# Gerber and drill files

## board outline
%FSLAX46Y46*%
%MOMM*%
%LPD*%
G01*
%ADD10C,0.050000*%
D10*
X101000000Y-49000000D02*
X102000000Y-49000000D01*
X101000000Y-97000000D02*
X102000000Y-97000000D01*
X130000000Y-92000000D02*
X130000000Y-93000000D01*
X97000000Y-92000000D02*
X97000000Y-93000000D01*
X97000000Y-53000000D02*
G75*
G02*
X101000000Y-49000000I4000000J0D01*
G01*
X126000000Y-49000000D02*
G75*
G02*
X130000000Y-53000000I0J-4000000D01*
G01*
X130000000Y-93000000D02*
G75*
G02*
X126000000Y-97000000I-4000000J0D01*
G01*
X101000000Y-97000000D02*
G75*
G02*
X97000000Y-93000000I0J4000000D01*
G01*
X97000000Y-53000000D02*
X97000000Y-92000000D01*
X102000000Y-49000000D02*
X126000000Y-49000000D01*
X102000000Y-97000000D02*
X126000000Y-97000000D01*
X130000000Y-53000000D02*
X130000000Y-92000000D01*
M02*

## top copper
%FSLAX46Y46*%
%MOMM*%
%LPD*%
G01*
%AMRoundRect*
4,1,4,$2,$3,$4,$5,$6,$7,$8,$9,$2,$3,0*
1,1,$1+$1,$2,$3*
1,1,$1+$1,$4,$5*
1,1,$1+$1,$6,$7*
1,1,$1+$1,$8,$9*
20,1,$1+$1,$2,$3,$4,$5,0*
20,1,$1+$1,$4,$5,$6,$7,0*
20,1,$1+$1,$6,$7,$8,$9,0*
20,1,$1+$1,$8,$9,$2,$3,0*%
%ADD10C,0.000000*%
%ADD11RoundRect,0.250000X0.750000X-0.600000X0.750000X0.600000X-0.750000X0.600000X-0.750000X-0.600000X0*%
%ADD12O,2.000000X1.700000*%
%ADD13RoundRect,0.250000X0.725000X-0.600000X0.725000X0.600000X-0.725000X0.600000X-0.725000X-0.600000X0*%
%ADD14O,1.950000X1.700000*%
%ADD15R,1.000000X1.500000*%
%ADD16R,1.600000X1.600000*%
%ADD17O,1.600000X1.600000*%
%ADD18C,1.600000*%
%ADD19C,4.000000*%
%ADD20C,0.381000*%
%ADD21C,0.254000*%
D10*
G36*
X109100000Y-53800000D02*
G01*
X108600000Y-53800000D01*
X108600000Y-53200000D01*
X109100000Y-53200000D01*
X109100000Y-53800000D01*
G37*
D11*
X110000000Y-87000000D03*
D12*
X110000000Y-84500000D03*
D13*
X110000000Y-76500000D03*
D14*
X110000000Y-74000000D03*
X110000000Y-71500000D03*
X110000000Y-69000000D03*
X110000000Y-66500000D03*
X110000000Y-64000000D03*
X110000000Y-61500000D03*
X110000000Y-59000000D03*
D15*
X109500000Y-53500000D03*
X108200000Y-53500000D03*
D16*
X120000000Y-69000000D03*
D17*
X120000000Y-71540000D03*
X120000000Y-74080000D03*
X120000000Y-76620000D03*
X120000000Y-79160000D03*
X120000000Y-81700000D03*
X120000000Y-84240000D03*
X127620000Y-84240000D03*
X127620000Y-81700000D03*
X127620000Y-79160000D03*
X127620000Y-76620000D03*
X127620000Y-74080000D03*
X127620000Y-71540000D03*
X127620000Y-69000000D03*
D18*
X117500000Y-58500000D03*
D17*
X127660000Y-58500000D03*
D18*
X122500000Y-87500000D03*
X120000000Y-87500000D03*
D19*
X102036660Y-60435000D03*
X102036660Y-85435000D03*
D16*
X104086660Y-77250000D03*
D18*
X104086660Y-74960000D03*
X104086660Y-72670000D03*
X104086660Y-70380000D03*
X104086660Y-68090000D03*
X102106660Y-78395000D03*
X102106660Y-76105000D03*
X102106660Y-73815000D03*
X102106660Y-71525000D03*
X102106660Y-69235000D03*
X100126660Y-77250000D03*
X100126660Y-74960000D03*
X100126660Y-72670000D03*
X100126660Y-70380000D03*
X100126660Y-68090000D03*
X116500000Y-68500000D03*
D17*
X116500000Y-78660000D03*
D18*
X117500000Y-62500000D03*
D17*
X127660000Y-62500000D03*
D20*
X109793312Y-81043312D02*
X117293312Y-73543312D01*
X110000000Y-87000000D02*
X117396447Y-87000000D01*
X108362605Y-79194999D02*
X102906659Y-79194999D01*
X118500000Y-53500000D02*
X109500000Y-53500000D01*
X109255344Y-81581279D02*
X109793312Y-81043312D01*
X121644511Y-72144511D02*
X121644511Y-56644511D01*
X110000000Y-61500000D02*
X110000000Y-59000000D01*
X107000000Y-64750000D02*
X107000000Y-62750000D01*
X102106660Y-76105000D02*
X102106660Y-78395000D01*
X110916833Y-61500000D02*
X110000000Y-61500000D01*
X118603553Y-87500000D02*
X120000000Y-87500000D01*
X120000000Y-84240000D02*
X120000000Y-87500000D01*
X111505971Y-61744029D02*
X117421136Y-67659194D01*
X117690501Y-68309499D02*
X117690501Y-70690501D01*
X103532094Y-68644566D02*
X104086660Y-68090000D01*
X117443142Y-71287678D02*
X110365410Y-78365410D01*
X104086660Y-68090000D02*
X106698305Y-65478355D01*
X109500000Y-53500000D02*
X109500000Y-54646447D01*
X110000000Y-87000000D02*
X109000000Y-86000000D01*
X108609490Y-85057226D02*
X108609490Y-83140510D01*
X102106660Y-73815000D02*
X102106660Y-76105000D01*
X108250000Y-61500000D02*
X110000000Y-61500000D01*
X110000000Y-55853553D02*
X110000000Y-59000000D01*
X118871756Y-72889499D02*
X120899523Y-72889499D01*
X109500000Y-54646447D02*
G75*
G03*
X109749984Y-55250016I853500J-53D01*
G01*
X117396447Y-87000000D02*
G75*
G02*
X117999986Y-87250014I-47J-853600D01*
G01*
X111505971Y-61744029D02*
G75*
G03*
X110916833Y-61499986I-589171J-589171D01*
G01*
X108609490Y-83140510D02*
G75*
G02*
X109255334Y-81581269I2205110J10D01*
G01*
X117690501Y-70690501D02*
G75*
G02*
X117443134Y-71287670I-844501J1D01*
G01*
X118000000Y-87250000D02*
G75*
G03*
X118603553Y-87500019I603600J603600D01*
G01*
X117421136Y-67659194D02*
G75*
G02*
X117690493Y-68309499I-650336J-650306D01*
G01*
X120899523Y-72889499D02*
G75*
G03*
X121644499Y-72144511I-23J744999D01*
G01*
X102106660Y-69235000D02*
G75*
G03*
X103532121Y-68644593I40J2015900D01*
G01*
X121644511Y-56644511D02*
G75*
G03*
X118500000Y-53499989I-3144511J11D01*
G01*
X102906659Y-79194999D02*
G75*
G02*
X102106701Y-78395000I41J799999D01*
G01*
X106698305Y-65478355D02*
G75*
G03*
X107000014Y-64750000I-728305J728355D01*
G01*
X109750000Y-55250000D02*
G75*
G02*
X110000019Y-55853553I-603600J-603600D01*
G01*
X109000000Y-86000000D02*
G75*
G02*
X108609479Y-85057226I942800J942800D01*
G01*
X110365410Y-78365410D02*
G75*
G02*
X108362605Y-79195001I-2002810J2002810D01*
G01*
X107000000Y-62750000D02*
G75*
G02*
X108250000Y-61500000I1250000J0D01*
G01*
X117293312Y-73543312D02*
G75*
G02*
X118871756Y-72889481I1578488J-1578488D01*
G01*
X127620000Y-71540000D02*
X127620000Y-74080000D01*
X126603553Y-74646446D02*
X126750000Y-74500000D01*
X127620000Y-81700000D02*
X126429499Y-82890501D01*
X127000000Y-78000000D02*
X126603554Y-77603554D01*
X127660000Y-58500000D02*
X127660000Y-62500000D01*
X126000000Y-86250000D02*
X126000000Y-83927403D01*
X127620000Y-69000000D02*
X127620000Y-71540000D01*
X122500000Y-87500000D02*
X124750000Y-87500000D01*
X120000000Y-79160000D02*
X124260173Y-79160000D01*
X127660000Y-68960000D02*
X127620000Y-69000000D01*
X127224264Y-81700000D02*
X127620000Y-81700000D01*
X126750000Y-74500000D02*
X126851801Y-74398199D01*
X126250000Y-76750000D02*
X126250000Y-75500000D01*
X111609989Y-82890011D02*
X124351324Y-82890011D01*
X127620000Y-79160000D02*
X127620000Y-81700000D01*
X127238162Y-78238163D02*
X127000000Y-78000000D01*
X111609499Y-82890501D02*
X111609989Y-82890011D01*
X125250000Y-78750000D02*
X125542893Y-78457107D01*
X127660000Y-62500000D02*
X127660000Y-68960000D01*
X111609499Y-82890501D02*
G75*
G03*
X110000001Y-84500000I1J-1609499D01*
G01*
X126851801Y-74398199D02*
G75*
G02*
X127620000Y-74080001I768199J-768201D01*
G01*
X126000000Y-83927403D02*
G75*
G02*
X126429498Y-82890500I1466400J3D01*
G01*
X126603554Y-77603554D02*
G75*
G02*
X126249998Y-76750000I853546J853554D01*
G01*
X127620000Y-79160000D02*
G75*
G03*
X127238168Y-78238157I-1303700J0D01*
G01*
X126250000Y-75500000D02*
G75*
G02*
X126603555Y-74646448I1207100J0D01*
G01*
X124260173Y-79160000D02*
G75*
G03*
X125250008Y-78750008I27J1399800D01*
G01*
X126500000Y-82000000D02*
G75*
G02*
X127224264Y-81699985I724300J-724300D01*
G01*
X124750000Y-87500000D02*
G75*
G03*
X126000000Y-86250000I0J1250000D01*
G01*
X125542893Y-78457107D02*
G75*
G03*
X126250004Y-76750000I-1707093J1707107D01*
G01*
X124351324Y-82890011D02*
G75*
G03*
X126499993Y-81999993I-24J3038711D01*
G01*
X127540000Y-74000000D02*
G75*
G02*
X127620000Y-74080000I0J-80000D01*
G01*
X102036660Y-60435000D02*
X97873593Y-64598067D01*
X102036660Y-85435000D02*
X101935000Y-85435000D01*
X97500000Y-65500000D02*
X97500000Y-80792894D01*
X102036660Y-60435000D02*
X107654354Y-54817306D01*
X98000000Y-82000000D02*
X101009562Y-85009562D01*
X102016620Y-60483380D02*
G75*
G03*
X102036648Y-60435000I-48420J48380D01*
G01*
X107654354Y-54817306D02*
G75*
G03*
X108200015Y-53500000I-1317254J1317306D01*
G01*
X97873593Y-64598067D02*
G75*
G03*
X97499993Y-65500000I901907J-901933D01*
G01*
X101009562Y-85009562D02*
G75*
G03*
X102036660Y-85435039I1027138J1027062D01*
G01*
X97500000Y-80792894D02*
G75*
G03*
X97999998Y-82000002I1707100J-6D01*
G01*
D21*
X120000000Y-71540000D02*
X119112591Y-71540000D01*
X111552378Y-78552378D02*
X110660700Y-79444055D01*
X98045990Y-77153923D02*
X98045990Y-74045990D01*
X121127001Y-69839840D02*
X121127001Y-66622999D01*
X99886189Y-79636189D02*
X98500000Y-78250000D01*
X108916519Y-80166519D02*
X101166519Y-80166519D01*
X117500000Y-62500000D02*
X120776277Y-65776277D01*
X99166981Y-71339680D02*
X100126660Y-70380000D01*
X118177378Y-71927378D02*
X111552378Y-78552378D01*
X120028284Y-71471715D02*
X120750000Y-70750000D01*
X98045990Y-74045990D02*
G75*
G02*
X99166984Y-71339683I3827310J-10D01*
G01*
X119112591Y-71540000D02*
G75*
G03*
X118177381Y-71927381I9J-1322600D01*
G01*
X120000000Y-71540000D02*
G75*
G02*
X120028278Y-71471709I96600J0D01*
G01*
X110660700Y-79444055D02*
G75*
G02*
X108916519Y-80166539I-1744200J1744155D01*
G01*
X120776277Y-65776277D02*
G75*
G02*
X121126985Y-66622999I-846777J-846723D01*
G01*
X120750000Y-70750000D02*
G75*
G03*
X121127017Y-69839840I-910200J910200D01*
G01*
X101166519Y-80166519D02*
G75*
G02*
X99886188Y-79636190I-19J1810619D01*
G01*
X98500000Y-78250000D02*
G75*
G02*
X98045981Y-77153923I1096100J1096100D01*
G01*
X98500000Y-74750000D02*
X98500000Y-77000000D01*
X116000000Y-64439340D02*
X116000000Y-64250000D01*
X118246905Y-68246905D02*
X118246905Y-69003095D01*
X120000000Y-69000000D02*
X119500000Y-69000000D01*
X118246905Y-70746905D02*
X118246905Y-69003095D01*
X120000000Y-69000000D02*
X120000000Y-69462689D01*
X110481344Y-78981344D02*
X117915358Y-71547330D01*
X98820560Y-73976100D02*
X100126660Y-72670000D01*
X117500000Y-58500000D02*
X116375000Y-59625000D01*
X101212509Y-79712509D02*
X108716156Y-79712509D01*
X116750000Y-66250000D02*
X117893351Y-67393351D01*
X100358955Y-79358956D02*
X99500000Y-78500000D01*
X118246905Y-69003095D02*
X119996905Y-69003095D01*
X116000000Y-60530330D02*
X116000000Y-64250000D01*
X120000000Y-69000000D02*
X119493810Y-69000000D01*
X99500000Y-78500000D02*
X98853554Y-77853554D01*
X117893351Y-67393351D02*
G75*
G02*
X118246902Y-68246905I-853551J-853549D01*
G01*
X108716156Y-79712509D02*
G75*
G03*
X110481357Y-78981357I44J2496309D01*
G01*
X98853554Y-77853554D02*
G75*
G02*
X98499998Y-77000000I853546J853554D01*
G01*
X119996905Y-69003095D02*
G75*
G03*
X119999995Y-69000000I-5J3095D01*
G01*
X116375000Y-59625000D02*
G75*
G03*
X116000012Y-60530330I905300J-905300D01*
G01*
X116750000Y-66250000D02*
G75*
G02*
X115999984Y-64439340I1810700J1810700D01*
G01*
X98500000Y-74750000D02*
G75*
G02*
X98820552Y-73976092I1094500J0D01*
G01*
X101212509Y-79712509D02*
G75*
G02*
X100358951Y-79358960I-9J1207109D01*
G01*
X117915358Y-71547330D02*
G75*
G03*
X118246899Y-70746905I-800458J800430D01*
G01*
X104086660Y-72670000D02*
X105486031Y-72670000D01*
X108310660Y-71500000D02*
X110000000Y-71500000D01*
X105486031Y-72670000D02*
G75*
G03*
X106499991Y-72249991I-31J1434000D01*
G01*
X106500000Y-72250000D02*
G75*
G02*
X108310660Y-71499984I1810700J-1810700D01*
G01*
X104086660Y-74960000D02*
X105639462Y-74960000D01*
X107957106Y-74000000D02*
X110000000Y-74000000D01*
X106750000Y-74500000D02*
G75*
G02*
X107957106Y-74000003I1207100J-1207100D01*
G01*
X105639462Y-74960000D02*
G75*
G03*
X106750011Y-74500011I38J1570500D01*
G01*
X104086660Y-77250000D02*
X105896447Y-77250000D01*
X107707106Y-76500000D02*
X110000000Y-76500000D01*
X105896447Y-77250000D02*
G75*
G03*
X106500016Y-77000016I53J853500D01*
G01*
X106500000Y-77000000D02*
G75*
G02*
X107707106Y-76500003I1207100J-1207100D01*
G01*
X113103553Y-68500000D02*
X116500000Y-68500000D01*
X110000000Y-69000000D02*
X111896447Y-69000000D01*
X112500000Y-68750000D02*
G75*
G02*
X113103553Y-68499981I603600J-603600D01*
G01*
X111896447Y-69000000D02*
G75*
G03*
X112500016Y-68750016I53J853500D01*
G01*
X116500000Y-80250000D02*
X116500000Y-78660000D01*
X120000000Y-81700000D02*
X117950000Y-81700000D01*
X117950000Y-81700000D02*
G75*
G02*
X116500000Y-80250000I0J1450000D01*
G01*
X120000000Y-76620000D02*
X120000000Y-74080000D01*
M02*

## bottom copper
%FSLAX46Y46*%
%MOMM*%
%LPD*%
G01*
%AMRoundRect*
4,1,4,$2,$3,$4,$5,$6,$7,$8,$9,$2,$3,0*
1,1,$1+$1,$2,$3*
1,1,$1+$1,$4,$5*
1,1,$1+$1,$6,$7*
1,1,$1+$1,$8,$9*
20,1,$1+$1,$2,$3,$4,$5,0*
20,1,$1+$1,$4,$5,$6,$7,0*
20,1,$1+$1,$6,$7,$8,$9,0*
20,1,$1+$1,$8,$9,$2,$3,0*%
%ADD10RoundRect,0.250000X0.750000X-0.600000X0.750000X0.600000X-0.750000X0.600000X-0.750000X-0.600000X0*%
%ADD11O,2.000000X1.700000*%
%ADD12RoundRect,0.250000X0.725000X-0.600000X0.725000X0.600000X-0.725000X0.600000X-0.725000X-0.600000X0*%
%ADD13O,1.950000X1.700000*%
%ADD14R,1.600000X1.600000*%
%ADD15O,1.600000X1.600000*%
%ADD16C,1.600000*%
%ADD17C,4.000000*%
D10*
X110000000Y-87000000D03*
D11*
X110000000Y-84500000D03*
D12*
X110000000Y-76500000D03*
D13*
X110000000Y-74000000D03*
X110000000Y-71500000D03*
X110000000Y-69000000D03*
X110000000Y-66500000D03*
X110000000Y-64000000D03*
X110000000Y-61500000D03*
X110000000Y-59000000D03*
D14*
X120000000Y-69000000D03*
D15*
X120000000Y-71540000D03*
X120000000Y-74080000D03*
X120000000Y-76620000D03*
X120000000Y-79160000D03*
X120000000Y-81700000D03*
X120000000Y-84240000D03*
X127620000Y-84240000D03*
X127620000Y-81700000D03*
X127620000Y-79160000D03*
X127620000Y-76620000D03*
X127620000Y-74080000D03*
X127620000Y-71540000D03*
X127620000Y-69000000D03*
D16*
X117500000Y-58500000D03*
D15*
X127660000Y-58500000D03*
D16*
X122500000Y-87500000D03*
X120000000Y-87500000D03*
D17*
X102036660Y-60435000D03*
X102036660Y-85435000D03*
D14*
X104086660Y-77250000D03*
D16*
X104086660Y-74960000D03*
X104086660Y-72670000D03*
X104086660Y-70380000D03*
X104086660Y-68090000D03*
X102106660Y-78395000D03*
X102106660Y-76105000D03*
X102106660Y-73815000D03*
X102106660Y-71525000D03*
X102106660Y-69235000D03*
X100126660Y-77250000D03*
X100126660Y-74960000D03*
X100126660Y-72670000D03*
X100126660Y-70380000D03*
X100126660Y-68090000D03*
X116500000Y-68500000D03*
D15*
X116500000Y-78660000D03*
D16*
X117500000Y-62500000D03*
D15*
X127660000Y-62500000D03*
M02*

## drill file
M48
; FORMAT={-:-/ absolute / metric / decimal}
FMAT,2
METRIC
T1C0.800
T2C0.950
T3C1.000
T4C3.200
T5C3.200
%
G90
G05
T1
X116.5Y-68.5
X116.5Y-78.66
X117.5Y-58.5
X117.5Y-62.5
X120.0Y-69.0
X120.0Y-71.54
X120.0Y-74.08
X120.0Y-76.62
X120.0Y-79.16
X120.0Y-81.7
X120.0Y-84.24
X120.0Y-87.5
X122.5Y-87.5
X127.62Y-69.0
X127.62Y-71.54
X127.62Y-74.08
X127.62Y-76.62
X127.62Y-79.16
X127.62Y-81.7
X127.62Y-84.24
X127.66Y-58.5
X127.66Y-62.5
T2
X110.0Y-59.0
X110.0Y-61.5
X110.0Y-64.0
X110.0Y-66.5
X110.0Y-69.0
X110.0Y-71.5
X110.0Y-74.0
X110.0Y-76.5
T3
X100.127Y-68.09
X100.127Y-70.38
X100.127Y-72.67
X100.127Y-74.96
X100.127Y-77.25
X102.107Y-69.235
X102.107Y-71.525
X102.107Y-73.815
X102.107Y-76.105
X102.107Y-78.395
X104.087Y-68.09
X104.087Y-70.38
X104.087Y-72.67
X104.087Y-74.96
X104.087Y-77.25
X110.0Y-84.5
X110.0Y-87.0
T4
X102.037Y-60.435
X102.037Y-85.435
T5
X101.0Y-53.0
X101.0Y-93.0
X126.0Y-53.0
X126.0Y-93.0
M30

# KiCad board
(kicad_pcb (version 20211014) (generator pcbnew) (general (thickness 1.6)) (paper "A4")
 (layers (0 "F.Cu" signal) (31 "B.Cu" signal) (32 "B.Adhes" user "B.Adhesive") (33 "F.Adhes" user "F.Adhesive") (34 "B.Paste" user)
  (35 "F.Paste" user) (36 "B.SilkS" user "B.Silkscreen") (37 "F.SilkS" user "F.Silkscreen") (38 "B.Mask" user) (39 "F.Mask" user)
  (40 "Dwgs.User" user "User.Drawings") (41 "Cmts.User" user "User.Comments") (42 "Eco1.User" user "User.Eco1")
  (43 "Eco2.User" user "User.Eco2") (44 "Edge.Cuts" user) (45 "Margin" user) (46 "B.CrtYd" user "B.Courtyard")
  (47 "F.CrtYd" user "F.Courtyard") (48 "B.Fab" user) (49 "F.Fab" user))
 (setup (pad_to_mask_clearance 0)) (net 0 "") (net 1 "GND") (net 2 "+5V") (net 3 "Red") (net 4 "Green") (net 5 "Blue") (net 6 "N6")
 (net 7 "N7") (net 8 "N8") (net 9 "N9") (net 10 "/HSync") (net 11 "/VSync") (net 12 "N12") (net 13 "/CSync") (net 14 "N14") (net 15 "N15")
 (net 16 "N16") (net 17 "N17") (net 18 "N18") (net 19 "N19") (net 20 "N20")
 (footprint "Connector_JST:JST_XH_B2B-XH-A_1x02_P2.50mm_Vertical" (layer "F.Cu") (at 110 87 90)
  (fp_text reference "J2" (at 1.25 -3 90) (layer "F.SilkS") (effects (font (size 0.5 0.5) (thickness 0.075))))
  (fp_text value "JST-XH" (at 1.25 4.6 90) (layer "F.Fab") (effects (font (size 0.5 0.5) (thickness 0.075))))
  (pad "1" thru_hole roundrect locked (at 0 0 90) (size 1.7 2) (drill 1) (layers *.Cu *.Mask) (roundrect_rratio 0.147059) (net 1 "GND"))
  (pad "2" thru_hole oval locked (at 2.5 0 90) (size 1.7 2) (drill 1) (layers *.Cu *.Mask) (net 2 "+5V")))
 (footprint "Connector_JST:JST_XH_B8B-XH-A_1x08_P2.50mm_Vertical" (layer "F.Cu") (at 110 76.5 90)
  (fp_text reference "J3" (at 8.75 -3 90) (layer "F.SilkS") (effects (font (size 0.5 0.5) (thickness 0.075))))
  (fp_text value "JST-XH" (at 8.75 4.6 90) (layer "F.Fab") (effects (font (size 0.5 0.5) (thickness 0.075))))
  (pad "1" thru_hole roundrect locked (at 0 0 90) (size 1.7 1.95) (drill 0.95) (layers *.Cu *.Mask) (roundrect_rratio 0.147059)
   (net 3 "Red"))
  (pad "2" thru_hole oval locked (at 2.5 0 90) (size 1.7 1.95) (drill 0.95) (layers *.Cu *.Mask) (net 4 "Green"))
  (pad "3" thru_hole oval locked (at 5 0 90) (size 1.7 1.95) (drill 0.95) (layers *.Cu *.Mask) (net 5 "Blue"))
  (pad "4" thru_hole oval locked (at 7.5 0 90) (size 1.7 1.95) (drill 0.95) (layers *.Cu *.Mask) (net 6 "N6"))
  (pad "5" thru_hole oval locked (at 10 0 90) (size 1.7 1.95) (drill 0.95) (layers *.Cu *.Mask) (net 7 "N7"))
  (pad "6" thru_hole oval locked (at 12.5 0 90) (size 1.7 1.95) (drill 0.95) (layers *.Cu *.Mask) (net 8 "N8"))
  (pad "7" thru_hole oval locked (at 15 0 90) (size 1.7 1.95) (drill 0.95) (layers *.Cu *.Mask) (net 1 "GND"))
  (pad "8" thru_hole oval locked (at 17.5 0 90) (size 1.7 1.95) (drill 0.95) (layers *.Cu *.Mask) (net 1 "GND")))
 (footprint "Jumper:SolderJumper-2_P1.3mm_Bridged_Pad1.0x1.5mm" (layer "F.Cu") (at 108.85 53.5 180)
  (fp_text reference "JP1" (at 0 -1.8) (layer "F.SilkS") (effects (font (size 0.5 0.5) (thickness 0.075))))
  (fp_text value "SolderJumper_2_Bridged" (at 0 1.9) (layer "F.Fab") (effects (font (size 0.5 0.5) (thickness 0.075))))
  (fp_poly (pts (xy -0.25 -0.3) (xy 0.25 -0.3) (xy 0.25 0.3) (xy -0.25 0.3)) (layer "F.Cu") (width 0) (fill solid))
  (pad "1" smd rect locked (at -0.65 0 180) (size 1 1.5) (layers "F.Cu" "F.Mask") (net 1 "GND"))
  (pad "2" smd rect locked (at 0.65 0 180) (size 1 1.5) (layers "F.Cu" "F.Mask") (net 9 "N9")))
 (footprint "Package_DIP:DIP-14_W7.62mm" (layer "F.Cu") (at 120 69)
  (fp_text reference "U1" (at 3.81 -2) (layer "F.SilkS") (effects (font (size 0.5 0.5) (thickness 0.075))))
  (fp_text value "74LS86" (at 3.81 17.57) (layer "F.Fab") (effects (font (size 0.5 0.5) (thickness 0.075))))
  (pad "1" thru_hole rect locked (at 0 0) (size 1.6 1.6) (drill 0.8) (layers *.Cu *.Mask) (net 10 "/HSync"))
  (pad "2" thru_hole oval locked (at 0 2.54) (size 1.6 1.6) (drill 0.8) (layers *.Cu *.Mask) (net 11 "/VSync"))
  (pad "3" thru_hole oval locked (at 0 5.08) (size 1.6 1.6) (drill 0.8) (layers *.Cu *.Mask) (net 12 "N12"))
  (pad "4" thru_hole oval locked (at 0 7.62) (size 1.6 1.6) (drill 0.8) (layers *.Cu *.Mask) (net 12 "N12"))
  (pad "5" thru_hole oval locked (at 0 10.16) (size 1.6 1.6) (drill 0.8) (layers *.Cu *.Mask) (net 2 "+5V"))
  (pad "6" thru_hole oval locked (at 0 12.7) (size 1.6 1.6) (drill 0.8) (layers *.Cu *.Mask) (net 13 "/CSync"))
  (pad "7" thru_hole oval locked (at 0 15.24) (size 1.6 1.6) (drill 0.8) (layers *.Cu *.Mask) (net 1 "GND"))
  (pad "8" thru_hole oval locked (at 7.62 15.24) (size 1.6 1.6) (drill 0.8) (layers *.Cu *.Mask) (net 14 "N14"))
  (pad "9" thru_hole oval locked (at 7.62 12.7) (size 1.6 1.6) (drill 0.8) (layers *.Cu *.Mask) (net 2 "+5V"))
  (pad "10" thru_hole oval locked (at 7.62 10.16) (size 1.6 1.6) (drill 0.8) (layers *.Cu *.Mask) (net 2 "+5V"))
  (pad "11" thru_hole oval locked (at 7.62 7.62) (size 1.6 1.6) (drill 0.8) (layers *.Cu *.Mask) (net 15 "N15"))
  (pad "12" thru_hole oval locked (at 7.62 5.08) (size 1.6 1.6) (drill 0.8) (layers *.Cu *.Mask) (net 2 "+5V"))
  (pad "13" thru_hole oval locked (at 7.62 2.54) (size 1.6 1.6) (drill 0.8) (layers *.Cu *.Mask) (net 2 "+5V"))
  (pad "14" thru_hole oval locked (at 7.62 0) (size 1.6 1.6) (drill 0.8) (layers *.Cu *.Mask) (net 2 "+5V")))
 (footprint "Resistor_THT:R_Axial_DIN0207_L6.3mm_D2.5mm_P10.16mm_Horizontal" (layer "F.Cu") (at 117.5 58.5)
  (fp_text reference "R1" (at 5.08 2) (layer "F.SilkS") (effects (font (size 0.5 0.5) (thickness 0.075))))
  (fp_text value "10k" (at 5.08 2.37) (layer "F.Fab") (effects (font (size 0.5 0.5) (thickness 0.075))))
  (pad "1" thru_hole circle locked (at 0 0) (size 1.6 1.6) (drill 0.8) (layers *.Cu *.Mask) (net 10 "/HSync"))
  (pad "2" thru_hole oval locked (at 10.16 0) (size 1.6 1.6) (drill 0.8) (layers *.Cu *.Mask) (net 2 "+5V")))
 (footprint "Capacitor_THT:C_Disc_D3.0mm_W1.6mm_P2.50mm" (layer "F.Cu") (at 122.5 87.5 180)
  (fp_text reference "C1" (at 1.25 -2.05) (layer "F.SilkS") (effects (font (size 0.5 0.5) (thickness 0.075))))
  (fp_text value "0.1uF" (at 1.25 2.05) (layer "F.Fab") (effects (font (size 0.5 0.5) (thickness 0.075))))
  (pad "1" thru_hole circle locked (at 0 0 180) (size 1.6 1.6) (drill 0.8) (layers *.Cu *.Mask) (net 2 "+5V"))
  (pad "2" thru_hole circle locked (at 2.5 0 180) (size 1.6 1.6) (drill 0.8) (layers *.Cu *.Mask) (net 1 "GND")))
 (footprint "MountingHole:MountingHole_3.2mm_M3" (layer "F.Cu") (at 101 53)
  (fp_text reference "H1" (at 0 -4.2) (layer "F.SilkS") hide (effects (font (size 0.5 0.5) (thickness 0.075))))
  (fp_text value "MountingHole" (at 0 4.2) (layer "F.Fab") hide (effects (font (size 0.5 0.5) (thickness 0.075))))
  (pad "" np_thru_hole circle locked (at 0 0) (size 3.2 3.2) (drill 3.2) (layers *.Cu *.Mask)))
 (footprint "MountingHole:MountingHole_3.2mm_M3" (layer "F.Cu") (at 101 93)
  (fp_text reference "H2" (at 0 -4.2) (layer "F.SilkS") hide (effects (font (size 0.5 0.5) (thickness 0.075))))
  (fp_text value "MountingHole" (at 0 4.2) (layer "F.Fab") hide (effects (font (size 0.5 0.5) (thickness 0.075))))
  (pad "" np_thru_hole circle locked (at 0 0) (size 3.2 3.2) (drill 3.2) (layers *.Cu *.Mask)))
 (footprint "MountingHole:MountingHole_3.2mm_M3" (layer "F.Cu") (at 126 93)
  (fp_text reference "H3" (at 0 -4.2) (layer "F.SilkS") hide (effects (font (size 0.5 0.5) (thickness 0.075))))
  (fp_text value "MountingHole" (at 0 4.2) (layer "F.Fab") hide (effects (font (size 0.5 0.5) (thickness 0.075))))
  (pad "" np_thru_hole circle locked (at 0 0) (size 3.2 3.2) (drill 3.2) (layers *.Cu *.Mask)))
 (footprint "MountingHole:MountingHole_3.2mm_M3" (layer "F.Cu") (at 126 53)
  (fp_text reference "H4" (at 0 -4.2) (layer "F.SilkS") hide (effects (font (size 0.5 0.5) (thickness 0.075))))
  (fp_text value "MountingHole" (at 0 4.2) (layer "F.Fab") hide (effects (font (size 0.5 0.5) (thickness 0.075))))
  (pad "" np_thru_hole circle locked (at 0 0) (size 3.2 3.2) (drill 3.2) (layers *.Cu *.Mask)))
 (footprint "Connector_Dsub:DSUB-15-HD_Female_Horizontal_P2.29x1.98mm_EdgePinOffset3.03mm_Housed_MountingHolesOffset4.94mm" (layer "F.Cu")
  (at 104.08666 77.25 -90)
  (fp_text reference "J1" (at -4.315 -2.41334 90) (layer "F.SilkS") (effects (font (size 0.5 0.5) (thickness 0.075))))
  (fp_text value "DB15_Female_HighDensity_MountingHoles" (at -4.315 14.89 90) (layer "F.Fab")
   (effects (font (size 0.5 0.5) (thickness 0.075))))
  (pad "0" thru_hole circle locked (at -16.815 2.05 270) (size 4 4) (drill 3.2) (layers *.Cu *.Mask) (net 9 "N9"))
  (pad "0" thru_hole circle locked (at 8.185 2.05 270) (size 4 4) (drill 3.2) (layers *.Cu *.Mask) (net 9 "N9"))
  (pad "1" thru_hole rect locked (at 0 0 270) (size 1.6 1.6) (drill 1) (layers *.Cu *.Mask) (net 3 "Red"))
  (pad "2" thru_hole circle locked (at -2.29 0 270) (size 1.6 1.6) (drill 1) (layers *.Cu *.Mask) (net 4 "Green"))
  (pad "3" thru_hole circle locked (at -4.58 0 270) (size 1.6 1.6) (drill 1) (layers *.Cu *.Mask) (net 5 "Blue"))
  (pad "4" thru_hole circle locked (at -6.87 0 270) (size 1.6 1.6) (drill 1) (layers *.Cu *.Mask) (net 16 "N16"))
  (pad "5" thru_hole circle locked (at -9.16 0 270) (size 1.6 1.6) (drill 1) (layers *.Cu *.Mask) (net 1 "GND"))
  (pad "6" thru_hole circle locked (at 1.145 1.98 270) (size 1.6 1.6) (drill 1) (layers *.Cu *.Mask) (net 1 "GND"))
  (pad "7" thru_hole circle locked (at -1.145 1.98 270) (size 1.6 1.6) (drill 1) (layers *.Cu *.Mask) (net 1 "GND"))
  (pad "8" thru_hole circle locked (at -3.435 1.98 270) (size 1.6 1.6) (drill 1) (layers *.Cu *.Mask) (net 1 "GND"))
  (pad "9" thru_hole circle locked (at -5.725 1.98 270) (size 1.6 1.6) (drill 1) (layers *.Cu *.Mask) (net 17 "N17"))
  (pad "10" thru_hole circle locked (at -8.015 1.98 270) (size 1.6 1.6) (drill 1) (layers *.Cu *.Mask) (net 1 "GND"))
  (pad "11" thru_hole circle locked (at 0 3.96 270) (size 1.6 1.6) (drill 1) (layers *.Cu *.Mask) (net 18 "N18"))
  (pad "12" thru_hole circle locked (at -2.29 3.96 270) (size 1.6 1.6) (drill 1) (layers *.Cu *.Mask) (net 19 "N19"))
  (pad "13" thru_hole circle locked (at -4.58 3.96 270) (size 1.6 1.6) (drill 1) (layers *.Cu *.Mask) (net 10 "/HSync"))
  (pad "14" thru_hole circle locked (at -6.87 3.96 270) (size 1.6 1.6) (drill 1) (layers *.Cu *.Mask) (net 11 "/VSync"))
  (pad "15" thru_hole circle locked (at -9.16 3.96 270) (size 1.6 1.6) (drill 1) (layers *.Cu *.Mask) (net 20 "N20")))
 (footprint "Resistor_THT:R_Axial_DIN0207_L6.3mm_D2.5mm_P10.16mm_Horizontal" (layer "F.Cu") (at 116.5 68.5 -90)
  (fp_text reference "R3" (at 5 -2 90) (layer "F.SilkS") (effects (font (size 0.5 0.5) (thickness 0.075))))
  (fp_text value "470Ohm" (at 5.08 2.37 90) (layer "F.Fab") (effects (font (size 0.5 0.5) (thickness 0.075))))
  (pad "1" thru_hole circle locked (at 0 0 270) (size 1.6 1.6) (drill 0.8) (layers *.Cu *.Mask) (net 6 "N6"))
  (pad "2" thru_hole oval locked (at 10.16 0 270) (size 1.6 1.6) (drill 0.8) (layers *.Cu *.Mask) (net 13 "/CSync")))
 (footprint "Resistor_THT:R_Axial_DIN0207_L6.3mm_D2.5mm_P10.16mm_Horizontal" (layer "F.Cu") (at 117.5 62.5)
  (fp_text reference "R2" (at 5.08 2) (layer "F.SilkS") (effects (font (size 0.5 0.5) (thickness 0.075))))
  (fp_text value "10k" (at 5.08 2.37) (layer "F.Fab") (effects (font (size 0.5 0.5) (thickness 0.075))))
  (pad "1" thru_hole circle locked (at 0 0) (size 1.6 1.6) (drill 0.8) (layers *.Cu *.Mask) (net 11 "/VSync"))
  (pad "2" thru_hole oval locked (at 10.16 0) (size 1.6 1.6) (drill 0.8) (layers *.Cu *.Mask) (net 2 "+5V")))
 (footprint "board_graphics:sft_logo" (layer "F.Cu") (at 107.5 93)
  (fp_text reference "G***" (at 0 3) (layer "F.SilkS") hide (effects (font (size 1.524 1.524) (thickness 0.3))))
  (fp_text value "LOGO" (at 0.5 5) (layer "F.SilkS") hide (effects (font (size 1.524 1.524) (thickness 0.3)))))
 (gr_line (start 101 49) (end 102 49) (layer "Edge.Cuts") (width 0.05))
 (gr_line (start 101 97) (end 102 97) (layer "Edge.Cuts") (width 0.05))
 (gr_line (start 130 92) (end 130 93) (layer "Edge.Cuts") (width 0.05))
 (gr_line (start 97 92) (end 97 93) (layer "Edge.Cuts") (width 0.05))
 (gr_arc (start 97 53) (mid 98.171573 50.171573) (end 101 49) (layer "Edge.Cuts") (width 0.05))
 (gr_arc (start 126 49) (mid 128.828427 50.171573) (end 130 53) (layer "Edge.Cuts") (width 0.05))
 (gr_arc (start 130 93) (mid 128.828427 95.828427) (end 126 97) (layer "Edge.Cuts") (width 0.05))
 (gr_arc (start 101 97) (mid 98.171573 95.828427) (end 97 93) (layer "Edge.Cuts") (width 0.05))
 (gr_line (start 97 53) (end 97 92) (layer "Edge.Cuts") (width 0.05))
 (gr_line (start 102 49) (end 126 49) (layer "Edge.Cuts") (width 0.05))
 (gr_line (start 102 97) (end 126 97) (layer "Edge.Cuts") (width 0.05))
 (gr_line (start 130 53) (end 130 92) (layer "Edge.Cuts") (width 0.05))
 (segment (start 109.793312 81.043312) (end 117.293312 73.543312) (width 0.381) (layer "F.Cu") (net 1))
 (segment (start 110 87) (end 117.396447 87) (width 0.381) (layer "F.Cu") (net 1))
 (segment (start 108.362605 79.194999) (end 102.906659 79.194999) (width 0.381) (layer "F.Cu") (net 1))
 (segment (start 118.5 53.5) (end 109.5 53.5) (width 0.381) (layer "F.Cu") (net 1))
 (segment (start 109.255344 81.581279) (end 109.793312 81.043312) (width 0.381) (layer "F.Cu") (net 1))
 (segment (start 121.644511 72.144511) (end 121.644511 56.644511) (width 0.381) (layer "F.Cu") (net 1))
 (segment (start 110 61.5) (end 110 59) (width 0.381) (layer "F.Cu") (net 1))
 (segment (start 107 64.75) (end 107 62.75) (width 0.381) (layer "F.Cu") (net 1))
 (segment (start 102.10666 76.105) (end 102.10666 78.395) (width 0.381) (layer "F.Cu") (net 1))
 (segment (start 110.916833 61.5) (end 110 61.5) (width 0.381) (layer "F.Cu") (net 1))
 (segment (start 118.603553 87.5) (end 120 87.5) (width 0.381) (layer "F.Cu") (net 1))
 (segment (start 120 84.24) (end 120 87.5) (width 0.381) (layer "F.Cu") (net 1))
 (segment (start 111.505971 61.744029) (end 117.421136 67.659194) (width 0.381) (layer "F.Cu") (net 1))
 (segment (start 117.690501 68.309499) (end 117.690501 70.690501) (width 0.381) (layer "F.Cu") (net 1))
 (segment (start 103.532094 68.644566) (end 104.08666 68.09) (width 0.381) (layer "F.Cu") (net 1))
 (segment (start 117.443142 71.287678) (end 110.36541 78.36541) (width 0.381) (layer "F.Cu") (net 1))
 (segment (start 104.08666 68.09) (end 106.698305 65.478355) (width 0.381) (layer "F.Cu") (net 1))
 (segment (start 109.5 53.5) (end 109.5 54.646447) (width 0.381) (layer "F.Cu") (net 1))
 (segment (start 110 87) (end 109 86) (width 0.381) (layer "F.Cu") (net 1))
 (segment (start 108.60949 85.057226) (end 108.60949 83.14051) (width 0.381) (layer "F.Cu") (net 1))
 (segment (start 102.10666 73.815) (end 102.10666 76.105) (width 0.381) (layer "F.Cu") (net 1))
 (segment (start 108.25 61.5) (end 110 61.5) (width 0.381) (layer "F.Cu") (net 1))
 (segment (start 110 55.853553) (end 110 59) (width 0.381) (layer "F.Cu") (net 1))
 (segment (start 118.871756 72.889499) (end 120.899523 72.889499) (width 0.381) (layer "F.Cu") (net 1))
 (arc (start 109.5 54.646447) (mid 109.564972 54.973087) (end 109.75 55.25) (width 0.381) (layer "F.Cu") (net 1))
 (arc (start 117.396447 87) (mid 117.723087 87.064973) (end 118 87.25) (width 0.381) (layer "F.Cu") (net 1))
 (arc (start 111.505971 61.744029) (mid 111.235673 61.563421) (end 110.916833 61.5) (width 0.381) (layer "F.Cu") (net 1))
 (arc (start 108.60949 83.14051) (mid 108.777342 82.296661) (end 109.255344 81.581279) (width 0.381) (layer "F.Cu") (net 1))
 (arc (start 117.690501 70.690501) (mid 117.626215 71.013692) (end 117.443142 71.287678) (width 0.381) (layer "F.Cu") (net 1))
 (arc (start 118 87.25) (mid 118.276912 87.435027) (end 118.603553 87.5) (width 0.381) (layer "F.Cu") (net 1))
 (arc (start 117.421136 67.659194) (mid 117.620495 67.957556) (end 117.690501 68.309499) (width 0.381) (layer "F.Cu") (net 1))
 (arc (start 120.899523 72.889499) (mid 121.426309 72.671297) (end 121.644511 72.144511) (width 0.381) (layer "F.Cu") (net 1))
 (arc (start 102.10666 69.235) (mid 102.878099 69.081551) (end 103.532094 68.644566) (width 0.381) (layer "F.Cu") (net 1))
 (arc (start 121.644511 56.644511) (mid 120.723505 54.421006) (end 118.5 53.5) (width 0.381) (layer "F.Cu") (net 1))
 (arc (start 102.906659 79.194999) (mid 102.340974 78.960685) (end 102.10666 78.395) (width 0.381) (layer "F.Cu") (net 1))
 (arc (start 106.698305 65.478355) (mid 106.921592 65.144184) (end 107 64.75) (width 0.381) (layer "F.Cu") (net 1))
 (arc (start 109.75 55.25) (mid 109.935027 55.526912) (end 110 55.853553) (width 0.381) (layer "F.Cu") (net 1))
 (arc (start 109 86) (mid 108.710981 85.567452) (end 108.60949 85.057226) (width 0.381) (layer "F.Cu") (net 1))
 (arc (start 110.36541 78.36541) (mid 109.446515 78.979396) (end 108.362605 79.194999) (width 0.381) (layer "F.Cu") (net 1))
 (arc (start 107 62.75) (mid 107.366117 61.866117) (end 108.25 61.5) (width 0.381) (layer "F.Cu") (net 1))
 (arc (start 117.293312 73.543312) (mid 118.017507 73.05942) (end 118.871756 72.889499) (width 0.381) (layer "F.Cu") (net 1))
 (segment (start 127.62 71.54) (end 127.62 74.08) (width 0.381) (layer "F.Cu") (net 2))
 (segment (start 126.603553 74.646446) (end 126.75 74.5) (width 0.381) (layer "F.Cu") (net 2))
 (segment (start 127.62 81.7) (end 126.429499 82.890501) (width 0.381) (layer "F.Cu") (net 2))
 (segment (start 127 78) (end 126.603554 77.603554) (width 0.381) (layer "F.Cu") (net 2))
 (segment (start 127.66 58.5) (end 127.66 62.5) (width 0.381) (layer "F.Cu") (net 2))
 (segment (start 126 86.25) (end 126 83.927403) (width 0.381) (layer "F.Cu") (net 2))
 (segment (start 127.62 69) (end 127.62 71.54) (width 0.381) (layer "F.Cu") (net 2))
 (segment (start 122.5 87.5) (end 124.75 87.5) (width 0.381) (layer "F.Cu") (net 2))
 (segment (start 120 79.16) (end 124.260173 79.16) (width 0.381) (layer "F.Cu") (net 2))
 (segment (start 127.66 68.96) (end 127.62 69) (width 0.381) (layer "F.Cu") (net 2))
 (segment (start 127.224264 81.7) (end 127.62 81.7) (width 0.381) (layer "F.Cu") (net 2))
 (segment (start 126.75 74.5) (end 126.851801 74.398199) (width 0.381) (layer "F.Cu") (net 2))
 (segment (start 126.25 76.75) (end 126.25 75.5) (width 0.381) (layer "F.Cu") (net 2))
 (segment (start 111.609989 82.890011) (end 124.351324 82.890011) (width 0.381) (layer "F.Cu") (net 2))
 (segment (start 127.62 79.16) (end 127.62 81.7) (width 0.381) (layer "F.Cu") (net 2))
 (segment (start 127.238162 78.238163) (end 127 78) (width 0.381) (layer "F.Cu") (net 2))
 (segment (start 111.609499 82.890501) (end 111.609989 82.890011) (width 0.381) (layer "F.Cu") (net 2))
 (segment (start 125.25 78.75) (end 125.542893 78.457107) (width 0.381) (layer "F.Cu") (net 2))
 (segment (start 127.66 62.5) (end 127.66 68.96) (width 0.381) (layer "F.Cu") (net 2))
 (arc (start 111.609499 82.890501) (mid 110.471411 83.361912) (end 110 84.5) (width 0.381) (layer "F.Cu") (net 2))
 (arc (start 126.851801 74.398199) (mid 127.204253 74.162698) (end 127.62 74.08) (width 0.381) (layer "F.Cu") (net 2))
 (arc (start 126 83.927403) (mid 126.111623 83.366236) (end 126.429499 82.890501) (width 0.381) (layer "F.Cu") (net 2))
 (arc (start 126.603554 77.603554) (mid 126.341886 77.21194) (end 126.25 76.75) (width 0.381) (layer "F.Cu") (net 2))
 (arc (start 127.62 79.16) (mid 127.520764 78.661105) (end 127.238162 78.238163) (width 0.381) (layer "F.Cu") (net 2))
 (arc (start 126.25 75.5) (mid 126.341886 75.03806) (end 126.603553 74.646446) (width 0.381) (layer "F.Cu") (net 2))
 (arc (start 124.260173 79.16) (mid 124.795863 79.053445) (end 125.25 78.75) (width 0.381) (layer "F.Cu") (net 2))
 (arc (start 126.5 82) (mid 126.832294 81.777968) (end 127.224264 81.7) (width 0.381) (layer "F.Cu") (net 2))
 (arc (start 124.75 87.5) (mid 125.633883 87.133883) (end 126 86.25) (width 0.381) (layer "F.Cu") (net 2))
 (arc (start 125.542893 78.457107) (mid 126.066229 77.67388) (end 126.25 76.75) (width 0.381) (layer "F.Cu") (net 2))
 (arc (start 124.351324 82.890011) (mid 125.514179 82.658705) (end 126.5 82) (width 0.381) (layer "F.Cu") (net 2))
 (arc (start 127.54 74) (mid 127.596569 74.023431) (end 127.62 74.08) (width 0.381) (layer "F.Cu") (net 2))
 (segment (start 102.03666 60.435) (end 97.873593 64.598067) (width 0.381) (layer "F.Cu") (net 9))
 (segment (start 102.03666 85.435) (end 101.935 85.435) (width 0.381) (layer "F.Cu") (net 9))
 (segment (start 97.5 65.5) (end 97.5 80.792894) (width 0.381) (layer "F.Cu") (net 9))
 (segment (start 102.03666 60.435) (end 107.654354 54.817306) (width 0.381) (layer "F.Cu") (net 9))
 (segment (start 98 82) (end 101.009562 85.009562) (width 0.381) (layer "F.Cu") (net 9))
 (arc (start 102.01662 60.48338) (mid 102.031452 60.461183) (end 102.03666 60.435) (width 0.381) (layer "F.Cu") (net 9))
 (arc (start 107.654354 54.817306) (mid 108.058191 54.212922) (end 108.2 53.5) (width 0.381) (layer "F.Cu") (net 9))
 (arc (start 97.873593 64.598067) (mid 97.597094 65.011877) (end 97.5 65.5) (width 0.381) (layer "F.Cu") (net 9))
 (arc (start 101.009562 85.009562) (mid 101.480798 85.324432) (end 102.03666 85.435) (width 0.381) (layer "F.Cu") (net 9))
 (arc (start 97.5 80.792894) (mid 97.629946 81.446175) (end 98 82) (width 0.381) (layer "F.Cu") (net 9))
 (segment (start 120 71.54) (end 119.112591 71.54) (width 0.254) (layer "F.Cu") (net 11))
 (segment (start 111.552378 78.552378) (end 110.6607 79.444055) (width 0.254) (layer "F.Cu") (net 11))
 (segment (start 98.04599 77.153923) (end 98.04599 74.04599) (width 0.254) (layer "F.Cu") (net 11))
 (segment (start 121.127001 69.83984) (end 121.127001 66.622999) (width 0.254) (layer "F.Cu") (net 11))
 (segment (start 99.886189 79.636189) (end 98.5 78.25) (width 0.254) (layer "F.Cu") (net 11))
 (segment (start 108.916519 80.166519) (end 101.166519 80.166519) (width 0.254) (layer "F.Cu") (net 11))
 (segment (start 117.5 62.5) (end 120.776277 65.776277) (width 0.254) (layer "F.Cu") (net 11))
 (segment (start 99.166981 71.33968) (end 100.12666 70.38) (width 0.254) (layer "F.Cu") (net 11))
 (segment (start 118.177378 71.927378) (end 111.552378 78.552378) (width 0.254) (layer "F.Cu") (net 11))
 (segment (start 120.028284 71.471715) (end 120.75 70.75) (width 0.254) (layer "F.Cu") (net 11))
 (arc (start 98.04599 74.04599) (mid 98.337326 72.581345) (end 99.166981 71.33968) (width 0.254) (layer "F.Cu") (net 11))
 (arc (start 119.112591 71.54) (mid 118.606457 71.640677) (end 118.177378 71.927378) (width 0.254) (layer "F.Cu") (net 11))
 (arc (start 120 71.54) (mid 120.007351 71.503045) (end 120.028284 71.471715) (width 0.254) (layer "F.Cu") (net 11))
 (arc (start 110.6607 79.444055) (mid 109.860463 79.978757) (end 108.916519 80.166519) (width 0.254) (layer "F.Cu") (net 11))
 (arc (start 120.776277 65.776277) (mid 121.03585 66.164756) (end 121.127001 66.622999) (width 0.254) (layer "F.Cu") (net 11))
 (arc (start 120.75 70.75) (mid 121.029021 70.332415) (end 121.127001 69.83984) (width 0.254) (layer "F.Cu") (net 11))
 (arc (start 101.166519 80.166519) (mid 100.473609 80.028691) (end 99.886189 79.636189) (width 0.254) (layer "F.Cu") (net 11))
 (arc (start 98.5 78.25) (mid 98.163984 77.747116) (end 98.04599 77.153923) (width 0.254) (layer "F.Cu") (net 11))
 (segment (start 98.5 74.75) (end 98.5 77) (width 0.254) (layer "F.Cu") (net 10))
 (segment (start 116 64.43934) (end 116 64.25) (width 0.254) (layer "F.Cu") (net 10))
 (segment (start 118.246905 68.246905) (end 118.246905 69.003095) (width 0.254) (layer "F.Cu") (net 10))
 (segment (start 120 69) (end 119.5 69) (width 0.254) (layer "F.Cu") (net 10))
 (segment (start 118.246905 70.746905) (end 118.246905 69.003095) (width 0.254) (layer "F.Cu") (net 10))
 (segment (start 120 69) (end 120 69.462689) (width 0.254) (layer "F.Cu") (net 10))
 (segment (start 110.481344 78.981344) (end 117.915358 71.54733) (width 0.254) (layer "F.Cu") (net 10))
 (segment (start 98.82056 73.9761) (end 100.12666 72.67) (width 0.254) (layer "F.Cu") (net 10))
 (segment (start 117.5 58.5) (end 116.375 59.625) (width 0.254) (layer "F.Cu") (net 10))
 (segment (start 101.212509 79.712509) (end 108.716156 79.712509) (width 0.254) (layer "F.Cu") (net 10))
 (segment (start 116.75 66.25) (end 117.893351 67.393351) (width 0.254) (layer "F.Cu") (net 10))
 (segment (start 100.358955 79.358956) (end 99.5 78.5) (width 0.254) (layer "F.Cu") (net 10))
 (segment (start 118.246905 69.003095) (end 119.996905 69.003095) (width 0.254) (layer "F.Cu") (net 10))
 (segment (start 116 60.53033) (end 116 64.25) (width 0.254) (layer "F.Cu") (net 10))
 (segment (start 120 69) (end 119.49381 69) (width 0.254) (layer "F.Cu") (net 10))
 (segment (start 99.5 78.5) (end 98.853554 77.853554) (width 0.254) (layer "F.Cu") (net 10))
 (arc (start 117.893351 67.393351) (mid 118.155019 67.784965) (end 118.246905 68.246905) (width 0.254) (layer "F.Cu") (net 10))
 (arc (start 108.716156 79.712509) (mid 109.671468 79.522486) (end 110.481344 78.981344) (width 0.254) (layer "F.Cu") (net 10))
 (arc (start 98.853554 77.853554) (mid 98.591886 77.46194) (end 98.5 77) (width 0.254) (layer "F.Cu") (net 10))
 (arc (start 119.996905 69.003095) (mid 119.999093 69.002188) (end 120 69) (width 0.254) (layer "F.Cu") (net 10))
 (arc (start 116.375 59.625) (mid 116.097459 60.040369) (end 116 60.53033) (width 0.254) (layer "F.Cu") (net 10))
 (arc (start 116.75 66.25) (mid 116.194919 65.419263) (end 116 64.43934) (width 0.254) (layer "F.Cu") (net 10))
 (arc (start 98.5 74.75) (mid 98.583311 74.331168) (end 98.82056 73.9761) (width 0.254) (layer "F.Cu") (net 10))
 (arc (start 101.212509 79.712509) (mid 100.750569 79.620623) (end 100.358955 79.358956) (width 0.254) (layer "F.Cu") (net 10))
 (arc (start 117.915358 71.54733) (mid 118.160739 71.180093) (end 118.246905 70.746905) (width 0.254) (layer "F.Cu") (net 10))
 (segment (start 104.08666 72.67) (end 105.486031 72.67) (width 0.254) (layer "F.Cu") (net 5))
 (segment (start 108.31066 71.5) (end 110 71.5) (width 0.254) (layer "F.Cu") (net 5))
 (arc (start 105.486031 72.67) (mid 106.034787 72.560846) (end 106.5 72.25) (width 0.254) (layer "F.Cu") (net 5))
 (arc (start 106.5 72.25) (mid 107.330737 71.694919) (end 108.31066 71.5) (width 0.254) (layer "F.Cu") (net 5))
 (segment (start 104.08666 74.96) (end 105.639462 74.96) (width 0.254) (layer "F.Cu") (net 4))
 (segment (start 107.957106 74) (end 110 74) (width 0.254) (layer "F.Cu") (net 4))
 (arc (start 106.75 74.5) (mid 107.303825 74.129946) (end 107.957106 74) (width 0.254) (layer "F.Cu") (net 4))
 (arc (start 105.639462 74.96) (mid 106.24048 74.840451) (end 106.75 74.5) (width 0.254) (layer "F.Cu") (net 4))
 (segment (start 104.08666 77.25) (end 105.896447 77.25) (width 0.254) (layer "F.Cu") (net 3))
 (segment (start 107.707106 76.5) (end 110 76.5) (width 0.254) (layer "F.Cu") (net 3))
 (arc (start 105.896447 77.25) (mid 106.223087 77.185028) (end 106.5 77) (width 0.254) (layer "F.Cu") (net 3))
 (arc (start 106.5 77) (mid 107.053825 76.629946) (end 107.707106 76.5) (width 0.254) (layer "F.Cu") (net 3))
 (segment (start 113.103553 68.5) (end 116.5 68.5) (width 0.254) (layer "F.Cu") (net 6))
 (segment (start 110 69) (end 111.896447 69) (width 0.254) (layer "F.Cu") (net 6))
 (arc (start 112.5 68.75) (mid 112.776912 68.564973) (end 113.103553 68.5) (width 0.254) (layer "F.Cu") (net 6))
 (arc (start 111.896447 69) (mid 112.223087 68.935028) (end 112.5 68.75) (width 0.254) (layer "F.Cu") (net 6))
 (segment (start 116.5 80.25) (end 116.5 78.66) (width 0.254) (layer "F.Cu") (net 13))
 (segment (start 120 81.7) (end 117.95 81.7) (width 0.254) (layer "F.Cu") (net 13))
 (arc (start 117.95 81.7) (mid 116.924695 81.275305) (end 116.5 80.25) (width 0.254) (layer "F.Cu") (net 13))
 (segment (start 120 76.62) (end 120 74.08) (width 0.254) (layer "F.Cu") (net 12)))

